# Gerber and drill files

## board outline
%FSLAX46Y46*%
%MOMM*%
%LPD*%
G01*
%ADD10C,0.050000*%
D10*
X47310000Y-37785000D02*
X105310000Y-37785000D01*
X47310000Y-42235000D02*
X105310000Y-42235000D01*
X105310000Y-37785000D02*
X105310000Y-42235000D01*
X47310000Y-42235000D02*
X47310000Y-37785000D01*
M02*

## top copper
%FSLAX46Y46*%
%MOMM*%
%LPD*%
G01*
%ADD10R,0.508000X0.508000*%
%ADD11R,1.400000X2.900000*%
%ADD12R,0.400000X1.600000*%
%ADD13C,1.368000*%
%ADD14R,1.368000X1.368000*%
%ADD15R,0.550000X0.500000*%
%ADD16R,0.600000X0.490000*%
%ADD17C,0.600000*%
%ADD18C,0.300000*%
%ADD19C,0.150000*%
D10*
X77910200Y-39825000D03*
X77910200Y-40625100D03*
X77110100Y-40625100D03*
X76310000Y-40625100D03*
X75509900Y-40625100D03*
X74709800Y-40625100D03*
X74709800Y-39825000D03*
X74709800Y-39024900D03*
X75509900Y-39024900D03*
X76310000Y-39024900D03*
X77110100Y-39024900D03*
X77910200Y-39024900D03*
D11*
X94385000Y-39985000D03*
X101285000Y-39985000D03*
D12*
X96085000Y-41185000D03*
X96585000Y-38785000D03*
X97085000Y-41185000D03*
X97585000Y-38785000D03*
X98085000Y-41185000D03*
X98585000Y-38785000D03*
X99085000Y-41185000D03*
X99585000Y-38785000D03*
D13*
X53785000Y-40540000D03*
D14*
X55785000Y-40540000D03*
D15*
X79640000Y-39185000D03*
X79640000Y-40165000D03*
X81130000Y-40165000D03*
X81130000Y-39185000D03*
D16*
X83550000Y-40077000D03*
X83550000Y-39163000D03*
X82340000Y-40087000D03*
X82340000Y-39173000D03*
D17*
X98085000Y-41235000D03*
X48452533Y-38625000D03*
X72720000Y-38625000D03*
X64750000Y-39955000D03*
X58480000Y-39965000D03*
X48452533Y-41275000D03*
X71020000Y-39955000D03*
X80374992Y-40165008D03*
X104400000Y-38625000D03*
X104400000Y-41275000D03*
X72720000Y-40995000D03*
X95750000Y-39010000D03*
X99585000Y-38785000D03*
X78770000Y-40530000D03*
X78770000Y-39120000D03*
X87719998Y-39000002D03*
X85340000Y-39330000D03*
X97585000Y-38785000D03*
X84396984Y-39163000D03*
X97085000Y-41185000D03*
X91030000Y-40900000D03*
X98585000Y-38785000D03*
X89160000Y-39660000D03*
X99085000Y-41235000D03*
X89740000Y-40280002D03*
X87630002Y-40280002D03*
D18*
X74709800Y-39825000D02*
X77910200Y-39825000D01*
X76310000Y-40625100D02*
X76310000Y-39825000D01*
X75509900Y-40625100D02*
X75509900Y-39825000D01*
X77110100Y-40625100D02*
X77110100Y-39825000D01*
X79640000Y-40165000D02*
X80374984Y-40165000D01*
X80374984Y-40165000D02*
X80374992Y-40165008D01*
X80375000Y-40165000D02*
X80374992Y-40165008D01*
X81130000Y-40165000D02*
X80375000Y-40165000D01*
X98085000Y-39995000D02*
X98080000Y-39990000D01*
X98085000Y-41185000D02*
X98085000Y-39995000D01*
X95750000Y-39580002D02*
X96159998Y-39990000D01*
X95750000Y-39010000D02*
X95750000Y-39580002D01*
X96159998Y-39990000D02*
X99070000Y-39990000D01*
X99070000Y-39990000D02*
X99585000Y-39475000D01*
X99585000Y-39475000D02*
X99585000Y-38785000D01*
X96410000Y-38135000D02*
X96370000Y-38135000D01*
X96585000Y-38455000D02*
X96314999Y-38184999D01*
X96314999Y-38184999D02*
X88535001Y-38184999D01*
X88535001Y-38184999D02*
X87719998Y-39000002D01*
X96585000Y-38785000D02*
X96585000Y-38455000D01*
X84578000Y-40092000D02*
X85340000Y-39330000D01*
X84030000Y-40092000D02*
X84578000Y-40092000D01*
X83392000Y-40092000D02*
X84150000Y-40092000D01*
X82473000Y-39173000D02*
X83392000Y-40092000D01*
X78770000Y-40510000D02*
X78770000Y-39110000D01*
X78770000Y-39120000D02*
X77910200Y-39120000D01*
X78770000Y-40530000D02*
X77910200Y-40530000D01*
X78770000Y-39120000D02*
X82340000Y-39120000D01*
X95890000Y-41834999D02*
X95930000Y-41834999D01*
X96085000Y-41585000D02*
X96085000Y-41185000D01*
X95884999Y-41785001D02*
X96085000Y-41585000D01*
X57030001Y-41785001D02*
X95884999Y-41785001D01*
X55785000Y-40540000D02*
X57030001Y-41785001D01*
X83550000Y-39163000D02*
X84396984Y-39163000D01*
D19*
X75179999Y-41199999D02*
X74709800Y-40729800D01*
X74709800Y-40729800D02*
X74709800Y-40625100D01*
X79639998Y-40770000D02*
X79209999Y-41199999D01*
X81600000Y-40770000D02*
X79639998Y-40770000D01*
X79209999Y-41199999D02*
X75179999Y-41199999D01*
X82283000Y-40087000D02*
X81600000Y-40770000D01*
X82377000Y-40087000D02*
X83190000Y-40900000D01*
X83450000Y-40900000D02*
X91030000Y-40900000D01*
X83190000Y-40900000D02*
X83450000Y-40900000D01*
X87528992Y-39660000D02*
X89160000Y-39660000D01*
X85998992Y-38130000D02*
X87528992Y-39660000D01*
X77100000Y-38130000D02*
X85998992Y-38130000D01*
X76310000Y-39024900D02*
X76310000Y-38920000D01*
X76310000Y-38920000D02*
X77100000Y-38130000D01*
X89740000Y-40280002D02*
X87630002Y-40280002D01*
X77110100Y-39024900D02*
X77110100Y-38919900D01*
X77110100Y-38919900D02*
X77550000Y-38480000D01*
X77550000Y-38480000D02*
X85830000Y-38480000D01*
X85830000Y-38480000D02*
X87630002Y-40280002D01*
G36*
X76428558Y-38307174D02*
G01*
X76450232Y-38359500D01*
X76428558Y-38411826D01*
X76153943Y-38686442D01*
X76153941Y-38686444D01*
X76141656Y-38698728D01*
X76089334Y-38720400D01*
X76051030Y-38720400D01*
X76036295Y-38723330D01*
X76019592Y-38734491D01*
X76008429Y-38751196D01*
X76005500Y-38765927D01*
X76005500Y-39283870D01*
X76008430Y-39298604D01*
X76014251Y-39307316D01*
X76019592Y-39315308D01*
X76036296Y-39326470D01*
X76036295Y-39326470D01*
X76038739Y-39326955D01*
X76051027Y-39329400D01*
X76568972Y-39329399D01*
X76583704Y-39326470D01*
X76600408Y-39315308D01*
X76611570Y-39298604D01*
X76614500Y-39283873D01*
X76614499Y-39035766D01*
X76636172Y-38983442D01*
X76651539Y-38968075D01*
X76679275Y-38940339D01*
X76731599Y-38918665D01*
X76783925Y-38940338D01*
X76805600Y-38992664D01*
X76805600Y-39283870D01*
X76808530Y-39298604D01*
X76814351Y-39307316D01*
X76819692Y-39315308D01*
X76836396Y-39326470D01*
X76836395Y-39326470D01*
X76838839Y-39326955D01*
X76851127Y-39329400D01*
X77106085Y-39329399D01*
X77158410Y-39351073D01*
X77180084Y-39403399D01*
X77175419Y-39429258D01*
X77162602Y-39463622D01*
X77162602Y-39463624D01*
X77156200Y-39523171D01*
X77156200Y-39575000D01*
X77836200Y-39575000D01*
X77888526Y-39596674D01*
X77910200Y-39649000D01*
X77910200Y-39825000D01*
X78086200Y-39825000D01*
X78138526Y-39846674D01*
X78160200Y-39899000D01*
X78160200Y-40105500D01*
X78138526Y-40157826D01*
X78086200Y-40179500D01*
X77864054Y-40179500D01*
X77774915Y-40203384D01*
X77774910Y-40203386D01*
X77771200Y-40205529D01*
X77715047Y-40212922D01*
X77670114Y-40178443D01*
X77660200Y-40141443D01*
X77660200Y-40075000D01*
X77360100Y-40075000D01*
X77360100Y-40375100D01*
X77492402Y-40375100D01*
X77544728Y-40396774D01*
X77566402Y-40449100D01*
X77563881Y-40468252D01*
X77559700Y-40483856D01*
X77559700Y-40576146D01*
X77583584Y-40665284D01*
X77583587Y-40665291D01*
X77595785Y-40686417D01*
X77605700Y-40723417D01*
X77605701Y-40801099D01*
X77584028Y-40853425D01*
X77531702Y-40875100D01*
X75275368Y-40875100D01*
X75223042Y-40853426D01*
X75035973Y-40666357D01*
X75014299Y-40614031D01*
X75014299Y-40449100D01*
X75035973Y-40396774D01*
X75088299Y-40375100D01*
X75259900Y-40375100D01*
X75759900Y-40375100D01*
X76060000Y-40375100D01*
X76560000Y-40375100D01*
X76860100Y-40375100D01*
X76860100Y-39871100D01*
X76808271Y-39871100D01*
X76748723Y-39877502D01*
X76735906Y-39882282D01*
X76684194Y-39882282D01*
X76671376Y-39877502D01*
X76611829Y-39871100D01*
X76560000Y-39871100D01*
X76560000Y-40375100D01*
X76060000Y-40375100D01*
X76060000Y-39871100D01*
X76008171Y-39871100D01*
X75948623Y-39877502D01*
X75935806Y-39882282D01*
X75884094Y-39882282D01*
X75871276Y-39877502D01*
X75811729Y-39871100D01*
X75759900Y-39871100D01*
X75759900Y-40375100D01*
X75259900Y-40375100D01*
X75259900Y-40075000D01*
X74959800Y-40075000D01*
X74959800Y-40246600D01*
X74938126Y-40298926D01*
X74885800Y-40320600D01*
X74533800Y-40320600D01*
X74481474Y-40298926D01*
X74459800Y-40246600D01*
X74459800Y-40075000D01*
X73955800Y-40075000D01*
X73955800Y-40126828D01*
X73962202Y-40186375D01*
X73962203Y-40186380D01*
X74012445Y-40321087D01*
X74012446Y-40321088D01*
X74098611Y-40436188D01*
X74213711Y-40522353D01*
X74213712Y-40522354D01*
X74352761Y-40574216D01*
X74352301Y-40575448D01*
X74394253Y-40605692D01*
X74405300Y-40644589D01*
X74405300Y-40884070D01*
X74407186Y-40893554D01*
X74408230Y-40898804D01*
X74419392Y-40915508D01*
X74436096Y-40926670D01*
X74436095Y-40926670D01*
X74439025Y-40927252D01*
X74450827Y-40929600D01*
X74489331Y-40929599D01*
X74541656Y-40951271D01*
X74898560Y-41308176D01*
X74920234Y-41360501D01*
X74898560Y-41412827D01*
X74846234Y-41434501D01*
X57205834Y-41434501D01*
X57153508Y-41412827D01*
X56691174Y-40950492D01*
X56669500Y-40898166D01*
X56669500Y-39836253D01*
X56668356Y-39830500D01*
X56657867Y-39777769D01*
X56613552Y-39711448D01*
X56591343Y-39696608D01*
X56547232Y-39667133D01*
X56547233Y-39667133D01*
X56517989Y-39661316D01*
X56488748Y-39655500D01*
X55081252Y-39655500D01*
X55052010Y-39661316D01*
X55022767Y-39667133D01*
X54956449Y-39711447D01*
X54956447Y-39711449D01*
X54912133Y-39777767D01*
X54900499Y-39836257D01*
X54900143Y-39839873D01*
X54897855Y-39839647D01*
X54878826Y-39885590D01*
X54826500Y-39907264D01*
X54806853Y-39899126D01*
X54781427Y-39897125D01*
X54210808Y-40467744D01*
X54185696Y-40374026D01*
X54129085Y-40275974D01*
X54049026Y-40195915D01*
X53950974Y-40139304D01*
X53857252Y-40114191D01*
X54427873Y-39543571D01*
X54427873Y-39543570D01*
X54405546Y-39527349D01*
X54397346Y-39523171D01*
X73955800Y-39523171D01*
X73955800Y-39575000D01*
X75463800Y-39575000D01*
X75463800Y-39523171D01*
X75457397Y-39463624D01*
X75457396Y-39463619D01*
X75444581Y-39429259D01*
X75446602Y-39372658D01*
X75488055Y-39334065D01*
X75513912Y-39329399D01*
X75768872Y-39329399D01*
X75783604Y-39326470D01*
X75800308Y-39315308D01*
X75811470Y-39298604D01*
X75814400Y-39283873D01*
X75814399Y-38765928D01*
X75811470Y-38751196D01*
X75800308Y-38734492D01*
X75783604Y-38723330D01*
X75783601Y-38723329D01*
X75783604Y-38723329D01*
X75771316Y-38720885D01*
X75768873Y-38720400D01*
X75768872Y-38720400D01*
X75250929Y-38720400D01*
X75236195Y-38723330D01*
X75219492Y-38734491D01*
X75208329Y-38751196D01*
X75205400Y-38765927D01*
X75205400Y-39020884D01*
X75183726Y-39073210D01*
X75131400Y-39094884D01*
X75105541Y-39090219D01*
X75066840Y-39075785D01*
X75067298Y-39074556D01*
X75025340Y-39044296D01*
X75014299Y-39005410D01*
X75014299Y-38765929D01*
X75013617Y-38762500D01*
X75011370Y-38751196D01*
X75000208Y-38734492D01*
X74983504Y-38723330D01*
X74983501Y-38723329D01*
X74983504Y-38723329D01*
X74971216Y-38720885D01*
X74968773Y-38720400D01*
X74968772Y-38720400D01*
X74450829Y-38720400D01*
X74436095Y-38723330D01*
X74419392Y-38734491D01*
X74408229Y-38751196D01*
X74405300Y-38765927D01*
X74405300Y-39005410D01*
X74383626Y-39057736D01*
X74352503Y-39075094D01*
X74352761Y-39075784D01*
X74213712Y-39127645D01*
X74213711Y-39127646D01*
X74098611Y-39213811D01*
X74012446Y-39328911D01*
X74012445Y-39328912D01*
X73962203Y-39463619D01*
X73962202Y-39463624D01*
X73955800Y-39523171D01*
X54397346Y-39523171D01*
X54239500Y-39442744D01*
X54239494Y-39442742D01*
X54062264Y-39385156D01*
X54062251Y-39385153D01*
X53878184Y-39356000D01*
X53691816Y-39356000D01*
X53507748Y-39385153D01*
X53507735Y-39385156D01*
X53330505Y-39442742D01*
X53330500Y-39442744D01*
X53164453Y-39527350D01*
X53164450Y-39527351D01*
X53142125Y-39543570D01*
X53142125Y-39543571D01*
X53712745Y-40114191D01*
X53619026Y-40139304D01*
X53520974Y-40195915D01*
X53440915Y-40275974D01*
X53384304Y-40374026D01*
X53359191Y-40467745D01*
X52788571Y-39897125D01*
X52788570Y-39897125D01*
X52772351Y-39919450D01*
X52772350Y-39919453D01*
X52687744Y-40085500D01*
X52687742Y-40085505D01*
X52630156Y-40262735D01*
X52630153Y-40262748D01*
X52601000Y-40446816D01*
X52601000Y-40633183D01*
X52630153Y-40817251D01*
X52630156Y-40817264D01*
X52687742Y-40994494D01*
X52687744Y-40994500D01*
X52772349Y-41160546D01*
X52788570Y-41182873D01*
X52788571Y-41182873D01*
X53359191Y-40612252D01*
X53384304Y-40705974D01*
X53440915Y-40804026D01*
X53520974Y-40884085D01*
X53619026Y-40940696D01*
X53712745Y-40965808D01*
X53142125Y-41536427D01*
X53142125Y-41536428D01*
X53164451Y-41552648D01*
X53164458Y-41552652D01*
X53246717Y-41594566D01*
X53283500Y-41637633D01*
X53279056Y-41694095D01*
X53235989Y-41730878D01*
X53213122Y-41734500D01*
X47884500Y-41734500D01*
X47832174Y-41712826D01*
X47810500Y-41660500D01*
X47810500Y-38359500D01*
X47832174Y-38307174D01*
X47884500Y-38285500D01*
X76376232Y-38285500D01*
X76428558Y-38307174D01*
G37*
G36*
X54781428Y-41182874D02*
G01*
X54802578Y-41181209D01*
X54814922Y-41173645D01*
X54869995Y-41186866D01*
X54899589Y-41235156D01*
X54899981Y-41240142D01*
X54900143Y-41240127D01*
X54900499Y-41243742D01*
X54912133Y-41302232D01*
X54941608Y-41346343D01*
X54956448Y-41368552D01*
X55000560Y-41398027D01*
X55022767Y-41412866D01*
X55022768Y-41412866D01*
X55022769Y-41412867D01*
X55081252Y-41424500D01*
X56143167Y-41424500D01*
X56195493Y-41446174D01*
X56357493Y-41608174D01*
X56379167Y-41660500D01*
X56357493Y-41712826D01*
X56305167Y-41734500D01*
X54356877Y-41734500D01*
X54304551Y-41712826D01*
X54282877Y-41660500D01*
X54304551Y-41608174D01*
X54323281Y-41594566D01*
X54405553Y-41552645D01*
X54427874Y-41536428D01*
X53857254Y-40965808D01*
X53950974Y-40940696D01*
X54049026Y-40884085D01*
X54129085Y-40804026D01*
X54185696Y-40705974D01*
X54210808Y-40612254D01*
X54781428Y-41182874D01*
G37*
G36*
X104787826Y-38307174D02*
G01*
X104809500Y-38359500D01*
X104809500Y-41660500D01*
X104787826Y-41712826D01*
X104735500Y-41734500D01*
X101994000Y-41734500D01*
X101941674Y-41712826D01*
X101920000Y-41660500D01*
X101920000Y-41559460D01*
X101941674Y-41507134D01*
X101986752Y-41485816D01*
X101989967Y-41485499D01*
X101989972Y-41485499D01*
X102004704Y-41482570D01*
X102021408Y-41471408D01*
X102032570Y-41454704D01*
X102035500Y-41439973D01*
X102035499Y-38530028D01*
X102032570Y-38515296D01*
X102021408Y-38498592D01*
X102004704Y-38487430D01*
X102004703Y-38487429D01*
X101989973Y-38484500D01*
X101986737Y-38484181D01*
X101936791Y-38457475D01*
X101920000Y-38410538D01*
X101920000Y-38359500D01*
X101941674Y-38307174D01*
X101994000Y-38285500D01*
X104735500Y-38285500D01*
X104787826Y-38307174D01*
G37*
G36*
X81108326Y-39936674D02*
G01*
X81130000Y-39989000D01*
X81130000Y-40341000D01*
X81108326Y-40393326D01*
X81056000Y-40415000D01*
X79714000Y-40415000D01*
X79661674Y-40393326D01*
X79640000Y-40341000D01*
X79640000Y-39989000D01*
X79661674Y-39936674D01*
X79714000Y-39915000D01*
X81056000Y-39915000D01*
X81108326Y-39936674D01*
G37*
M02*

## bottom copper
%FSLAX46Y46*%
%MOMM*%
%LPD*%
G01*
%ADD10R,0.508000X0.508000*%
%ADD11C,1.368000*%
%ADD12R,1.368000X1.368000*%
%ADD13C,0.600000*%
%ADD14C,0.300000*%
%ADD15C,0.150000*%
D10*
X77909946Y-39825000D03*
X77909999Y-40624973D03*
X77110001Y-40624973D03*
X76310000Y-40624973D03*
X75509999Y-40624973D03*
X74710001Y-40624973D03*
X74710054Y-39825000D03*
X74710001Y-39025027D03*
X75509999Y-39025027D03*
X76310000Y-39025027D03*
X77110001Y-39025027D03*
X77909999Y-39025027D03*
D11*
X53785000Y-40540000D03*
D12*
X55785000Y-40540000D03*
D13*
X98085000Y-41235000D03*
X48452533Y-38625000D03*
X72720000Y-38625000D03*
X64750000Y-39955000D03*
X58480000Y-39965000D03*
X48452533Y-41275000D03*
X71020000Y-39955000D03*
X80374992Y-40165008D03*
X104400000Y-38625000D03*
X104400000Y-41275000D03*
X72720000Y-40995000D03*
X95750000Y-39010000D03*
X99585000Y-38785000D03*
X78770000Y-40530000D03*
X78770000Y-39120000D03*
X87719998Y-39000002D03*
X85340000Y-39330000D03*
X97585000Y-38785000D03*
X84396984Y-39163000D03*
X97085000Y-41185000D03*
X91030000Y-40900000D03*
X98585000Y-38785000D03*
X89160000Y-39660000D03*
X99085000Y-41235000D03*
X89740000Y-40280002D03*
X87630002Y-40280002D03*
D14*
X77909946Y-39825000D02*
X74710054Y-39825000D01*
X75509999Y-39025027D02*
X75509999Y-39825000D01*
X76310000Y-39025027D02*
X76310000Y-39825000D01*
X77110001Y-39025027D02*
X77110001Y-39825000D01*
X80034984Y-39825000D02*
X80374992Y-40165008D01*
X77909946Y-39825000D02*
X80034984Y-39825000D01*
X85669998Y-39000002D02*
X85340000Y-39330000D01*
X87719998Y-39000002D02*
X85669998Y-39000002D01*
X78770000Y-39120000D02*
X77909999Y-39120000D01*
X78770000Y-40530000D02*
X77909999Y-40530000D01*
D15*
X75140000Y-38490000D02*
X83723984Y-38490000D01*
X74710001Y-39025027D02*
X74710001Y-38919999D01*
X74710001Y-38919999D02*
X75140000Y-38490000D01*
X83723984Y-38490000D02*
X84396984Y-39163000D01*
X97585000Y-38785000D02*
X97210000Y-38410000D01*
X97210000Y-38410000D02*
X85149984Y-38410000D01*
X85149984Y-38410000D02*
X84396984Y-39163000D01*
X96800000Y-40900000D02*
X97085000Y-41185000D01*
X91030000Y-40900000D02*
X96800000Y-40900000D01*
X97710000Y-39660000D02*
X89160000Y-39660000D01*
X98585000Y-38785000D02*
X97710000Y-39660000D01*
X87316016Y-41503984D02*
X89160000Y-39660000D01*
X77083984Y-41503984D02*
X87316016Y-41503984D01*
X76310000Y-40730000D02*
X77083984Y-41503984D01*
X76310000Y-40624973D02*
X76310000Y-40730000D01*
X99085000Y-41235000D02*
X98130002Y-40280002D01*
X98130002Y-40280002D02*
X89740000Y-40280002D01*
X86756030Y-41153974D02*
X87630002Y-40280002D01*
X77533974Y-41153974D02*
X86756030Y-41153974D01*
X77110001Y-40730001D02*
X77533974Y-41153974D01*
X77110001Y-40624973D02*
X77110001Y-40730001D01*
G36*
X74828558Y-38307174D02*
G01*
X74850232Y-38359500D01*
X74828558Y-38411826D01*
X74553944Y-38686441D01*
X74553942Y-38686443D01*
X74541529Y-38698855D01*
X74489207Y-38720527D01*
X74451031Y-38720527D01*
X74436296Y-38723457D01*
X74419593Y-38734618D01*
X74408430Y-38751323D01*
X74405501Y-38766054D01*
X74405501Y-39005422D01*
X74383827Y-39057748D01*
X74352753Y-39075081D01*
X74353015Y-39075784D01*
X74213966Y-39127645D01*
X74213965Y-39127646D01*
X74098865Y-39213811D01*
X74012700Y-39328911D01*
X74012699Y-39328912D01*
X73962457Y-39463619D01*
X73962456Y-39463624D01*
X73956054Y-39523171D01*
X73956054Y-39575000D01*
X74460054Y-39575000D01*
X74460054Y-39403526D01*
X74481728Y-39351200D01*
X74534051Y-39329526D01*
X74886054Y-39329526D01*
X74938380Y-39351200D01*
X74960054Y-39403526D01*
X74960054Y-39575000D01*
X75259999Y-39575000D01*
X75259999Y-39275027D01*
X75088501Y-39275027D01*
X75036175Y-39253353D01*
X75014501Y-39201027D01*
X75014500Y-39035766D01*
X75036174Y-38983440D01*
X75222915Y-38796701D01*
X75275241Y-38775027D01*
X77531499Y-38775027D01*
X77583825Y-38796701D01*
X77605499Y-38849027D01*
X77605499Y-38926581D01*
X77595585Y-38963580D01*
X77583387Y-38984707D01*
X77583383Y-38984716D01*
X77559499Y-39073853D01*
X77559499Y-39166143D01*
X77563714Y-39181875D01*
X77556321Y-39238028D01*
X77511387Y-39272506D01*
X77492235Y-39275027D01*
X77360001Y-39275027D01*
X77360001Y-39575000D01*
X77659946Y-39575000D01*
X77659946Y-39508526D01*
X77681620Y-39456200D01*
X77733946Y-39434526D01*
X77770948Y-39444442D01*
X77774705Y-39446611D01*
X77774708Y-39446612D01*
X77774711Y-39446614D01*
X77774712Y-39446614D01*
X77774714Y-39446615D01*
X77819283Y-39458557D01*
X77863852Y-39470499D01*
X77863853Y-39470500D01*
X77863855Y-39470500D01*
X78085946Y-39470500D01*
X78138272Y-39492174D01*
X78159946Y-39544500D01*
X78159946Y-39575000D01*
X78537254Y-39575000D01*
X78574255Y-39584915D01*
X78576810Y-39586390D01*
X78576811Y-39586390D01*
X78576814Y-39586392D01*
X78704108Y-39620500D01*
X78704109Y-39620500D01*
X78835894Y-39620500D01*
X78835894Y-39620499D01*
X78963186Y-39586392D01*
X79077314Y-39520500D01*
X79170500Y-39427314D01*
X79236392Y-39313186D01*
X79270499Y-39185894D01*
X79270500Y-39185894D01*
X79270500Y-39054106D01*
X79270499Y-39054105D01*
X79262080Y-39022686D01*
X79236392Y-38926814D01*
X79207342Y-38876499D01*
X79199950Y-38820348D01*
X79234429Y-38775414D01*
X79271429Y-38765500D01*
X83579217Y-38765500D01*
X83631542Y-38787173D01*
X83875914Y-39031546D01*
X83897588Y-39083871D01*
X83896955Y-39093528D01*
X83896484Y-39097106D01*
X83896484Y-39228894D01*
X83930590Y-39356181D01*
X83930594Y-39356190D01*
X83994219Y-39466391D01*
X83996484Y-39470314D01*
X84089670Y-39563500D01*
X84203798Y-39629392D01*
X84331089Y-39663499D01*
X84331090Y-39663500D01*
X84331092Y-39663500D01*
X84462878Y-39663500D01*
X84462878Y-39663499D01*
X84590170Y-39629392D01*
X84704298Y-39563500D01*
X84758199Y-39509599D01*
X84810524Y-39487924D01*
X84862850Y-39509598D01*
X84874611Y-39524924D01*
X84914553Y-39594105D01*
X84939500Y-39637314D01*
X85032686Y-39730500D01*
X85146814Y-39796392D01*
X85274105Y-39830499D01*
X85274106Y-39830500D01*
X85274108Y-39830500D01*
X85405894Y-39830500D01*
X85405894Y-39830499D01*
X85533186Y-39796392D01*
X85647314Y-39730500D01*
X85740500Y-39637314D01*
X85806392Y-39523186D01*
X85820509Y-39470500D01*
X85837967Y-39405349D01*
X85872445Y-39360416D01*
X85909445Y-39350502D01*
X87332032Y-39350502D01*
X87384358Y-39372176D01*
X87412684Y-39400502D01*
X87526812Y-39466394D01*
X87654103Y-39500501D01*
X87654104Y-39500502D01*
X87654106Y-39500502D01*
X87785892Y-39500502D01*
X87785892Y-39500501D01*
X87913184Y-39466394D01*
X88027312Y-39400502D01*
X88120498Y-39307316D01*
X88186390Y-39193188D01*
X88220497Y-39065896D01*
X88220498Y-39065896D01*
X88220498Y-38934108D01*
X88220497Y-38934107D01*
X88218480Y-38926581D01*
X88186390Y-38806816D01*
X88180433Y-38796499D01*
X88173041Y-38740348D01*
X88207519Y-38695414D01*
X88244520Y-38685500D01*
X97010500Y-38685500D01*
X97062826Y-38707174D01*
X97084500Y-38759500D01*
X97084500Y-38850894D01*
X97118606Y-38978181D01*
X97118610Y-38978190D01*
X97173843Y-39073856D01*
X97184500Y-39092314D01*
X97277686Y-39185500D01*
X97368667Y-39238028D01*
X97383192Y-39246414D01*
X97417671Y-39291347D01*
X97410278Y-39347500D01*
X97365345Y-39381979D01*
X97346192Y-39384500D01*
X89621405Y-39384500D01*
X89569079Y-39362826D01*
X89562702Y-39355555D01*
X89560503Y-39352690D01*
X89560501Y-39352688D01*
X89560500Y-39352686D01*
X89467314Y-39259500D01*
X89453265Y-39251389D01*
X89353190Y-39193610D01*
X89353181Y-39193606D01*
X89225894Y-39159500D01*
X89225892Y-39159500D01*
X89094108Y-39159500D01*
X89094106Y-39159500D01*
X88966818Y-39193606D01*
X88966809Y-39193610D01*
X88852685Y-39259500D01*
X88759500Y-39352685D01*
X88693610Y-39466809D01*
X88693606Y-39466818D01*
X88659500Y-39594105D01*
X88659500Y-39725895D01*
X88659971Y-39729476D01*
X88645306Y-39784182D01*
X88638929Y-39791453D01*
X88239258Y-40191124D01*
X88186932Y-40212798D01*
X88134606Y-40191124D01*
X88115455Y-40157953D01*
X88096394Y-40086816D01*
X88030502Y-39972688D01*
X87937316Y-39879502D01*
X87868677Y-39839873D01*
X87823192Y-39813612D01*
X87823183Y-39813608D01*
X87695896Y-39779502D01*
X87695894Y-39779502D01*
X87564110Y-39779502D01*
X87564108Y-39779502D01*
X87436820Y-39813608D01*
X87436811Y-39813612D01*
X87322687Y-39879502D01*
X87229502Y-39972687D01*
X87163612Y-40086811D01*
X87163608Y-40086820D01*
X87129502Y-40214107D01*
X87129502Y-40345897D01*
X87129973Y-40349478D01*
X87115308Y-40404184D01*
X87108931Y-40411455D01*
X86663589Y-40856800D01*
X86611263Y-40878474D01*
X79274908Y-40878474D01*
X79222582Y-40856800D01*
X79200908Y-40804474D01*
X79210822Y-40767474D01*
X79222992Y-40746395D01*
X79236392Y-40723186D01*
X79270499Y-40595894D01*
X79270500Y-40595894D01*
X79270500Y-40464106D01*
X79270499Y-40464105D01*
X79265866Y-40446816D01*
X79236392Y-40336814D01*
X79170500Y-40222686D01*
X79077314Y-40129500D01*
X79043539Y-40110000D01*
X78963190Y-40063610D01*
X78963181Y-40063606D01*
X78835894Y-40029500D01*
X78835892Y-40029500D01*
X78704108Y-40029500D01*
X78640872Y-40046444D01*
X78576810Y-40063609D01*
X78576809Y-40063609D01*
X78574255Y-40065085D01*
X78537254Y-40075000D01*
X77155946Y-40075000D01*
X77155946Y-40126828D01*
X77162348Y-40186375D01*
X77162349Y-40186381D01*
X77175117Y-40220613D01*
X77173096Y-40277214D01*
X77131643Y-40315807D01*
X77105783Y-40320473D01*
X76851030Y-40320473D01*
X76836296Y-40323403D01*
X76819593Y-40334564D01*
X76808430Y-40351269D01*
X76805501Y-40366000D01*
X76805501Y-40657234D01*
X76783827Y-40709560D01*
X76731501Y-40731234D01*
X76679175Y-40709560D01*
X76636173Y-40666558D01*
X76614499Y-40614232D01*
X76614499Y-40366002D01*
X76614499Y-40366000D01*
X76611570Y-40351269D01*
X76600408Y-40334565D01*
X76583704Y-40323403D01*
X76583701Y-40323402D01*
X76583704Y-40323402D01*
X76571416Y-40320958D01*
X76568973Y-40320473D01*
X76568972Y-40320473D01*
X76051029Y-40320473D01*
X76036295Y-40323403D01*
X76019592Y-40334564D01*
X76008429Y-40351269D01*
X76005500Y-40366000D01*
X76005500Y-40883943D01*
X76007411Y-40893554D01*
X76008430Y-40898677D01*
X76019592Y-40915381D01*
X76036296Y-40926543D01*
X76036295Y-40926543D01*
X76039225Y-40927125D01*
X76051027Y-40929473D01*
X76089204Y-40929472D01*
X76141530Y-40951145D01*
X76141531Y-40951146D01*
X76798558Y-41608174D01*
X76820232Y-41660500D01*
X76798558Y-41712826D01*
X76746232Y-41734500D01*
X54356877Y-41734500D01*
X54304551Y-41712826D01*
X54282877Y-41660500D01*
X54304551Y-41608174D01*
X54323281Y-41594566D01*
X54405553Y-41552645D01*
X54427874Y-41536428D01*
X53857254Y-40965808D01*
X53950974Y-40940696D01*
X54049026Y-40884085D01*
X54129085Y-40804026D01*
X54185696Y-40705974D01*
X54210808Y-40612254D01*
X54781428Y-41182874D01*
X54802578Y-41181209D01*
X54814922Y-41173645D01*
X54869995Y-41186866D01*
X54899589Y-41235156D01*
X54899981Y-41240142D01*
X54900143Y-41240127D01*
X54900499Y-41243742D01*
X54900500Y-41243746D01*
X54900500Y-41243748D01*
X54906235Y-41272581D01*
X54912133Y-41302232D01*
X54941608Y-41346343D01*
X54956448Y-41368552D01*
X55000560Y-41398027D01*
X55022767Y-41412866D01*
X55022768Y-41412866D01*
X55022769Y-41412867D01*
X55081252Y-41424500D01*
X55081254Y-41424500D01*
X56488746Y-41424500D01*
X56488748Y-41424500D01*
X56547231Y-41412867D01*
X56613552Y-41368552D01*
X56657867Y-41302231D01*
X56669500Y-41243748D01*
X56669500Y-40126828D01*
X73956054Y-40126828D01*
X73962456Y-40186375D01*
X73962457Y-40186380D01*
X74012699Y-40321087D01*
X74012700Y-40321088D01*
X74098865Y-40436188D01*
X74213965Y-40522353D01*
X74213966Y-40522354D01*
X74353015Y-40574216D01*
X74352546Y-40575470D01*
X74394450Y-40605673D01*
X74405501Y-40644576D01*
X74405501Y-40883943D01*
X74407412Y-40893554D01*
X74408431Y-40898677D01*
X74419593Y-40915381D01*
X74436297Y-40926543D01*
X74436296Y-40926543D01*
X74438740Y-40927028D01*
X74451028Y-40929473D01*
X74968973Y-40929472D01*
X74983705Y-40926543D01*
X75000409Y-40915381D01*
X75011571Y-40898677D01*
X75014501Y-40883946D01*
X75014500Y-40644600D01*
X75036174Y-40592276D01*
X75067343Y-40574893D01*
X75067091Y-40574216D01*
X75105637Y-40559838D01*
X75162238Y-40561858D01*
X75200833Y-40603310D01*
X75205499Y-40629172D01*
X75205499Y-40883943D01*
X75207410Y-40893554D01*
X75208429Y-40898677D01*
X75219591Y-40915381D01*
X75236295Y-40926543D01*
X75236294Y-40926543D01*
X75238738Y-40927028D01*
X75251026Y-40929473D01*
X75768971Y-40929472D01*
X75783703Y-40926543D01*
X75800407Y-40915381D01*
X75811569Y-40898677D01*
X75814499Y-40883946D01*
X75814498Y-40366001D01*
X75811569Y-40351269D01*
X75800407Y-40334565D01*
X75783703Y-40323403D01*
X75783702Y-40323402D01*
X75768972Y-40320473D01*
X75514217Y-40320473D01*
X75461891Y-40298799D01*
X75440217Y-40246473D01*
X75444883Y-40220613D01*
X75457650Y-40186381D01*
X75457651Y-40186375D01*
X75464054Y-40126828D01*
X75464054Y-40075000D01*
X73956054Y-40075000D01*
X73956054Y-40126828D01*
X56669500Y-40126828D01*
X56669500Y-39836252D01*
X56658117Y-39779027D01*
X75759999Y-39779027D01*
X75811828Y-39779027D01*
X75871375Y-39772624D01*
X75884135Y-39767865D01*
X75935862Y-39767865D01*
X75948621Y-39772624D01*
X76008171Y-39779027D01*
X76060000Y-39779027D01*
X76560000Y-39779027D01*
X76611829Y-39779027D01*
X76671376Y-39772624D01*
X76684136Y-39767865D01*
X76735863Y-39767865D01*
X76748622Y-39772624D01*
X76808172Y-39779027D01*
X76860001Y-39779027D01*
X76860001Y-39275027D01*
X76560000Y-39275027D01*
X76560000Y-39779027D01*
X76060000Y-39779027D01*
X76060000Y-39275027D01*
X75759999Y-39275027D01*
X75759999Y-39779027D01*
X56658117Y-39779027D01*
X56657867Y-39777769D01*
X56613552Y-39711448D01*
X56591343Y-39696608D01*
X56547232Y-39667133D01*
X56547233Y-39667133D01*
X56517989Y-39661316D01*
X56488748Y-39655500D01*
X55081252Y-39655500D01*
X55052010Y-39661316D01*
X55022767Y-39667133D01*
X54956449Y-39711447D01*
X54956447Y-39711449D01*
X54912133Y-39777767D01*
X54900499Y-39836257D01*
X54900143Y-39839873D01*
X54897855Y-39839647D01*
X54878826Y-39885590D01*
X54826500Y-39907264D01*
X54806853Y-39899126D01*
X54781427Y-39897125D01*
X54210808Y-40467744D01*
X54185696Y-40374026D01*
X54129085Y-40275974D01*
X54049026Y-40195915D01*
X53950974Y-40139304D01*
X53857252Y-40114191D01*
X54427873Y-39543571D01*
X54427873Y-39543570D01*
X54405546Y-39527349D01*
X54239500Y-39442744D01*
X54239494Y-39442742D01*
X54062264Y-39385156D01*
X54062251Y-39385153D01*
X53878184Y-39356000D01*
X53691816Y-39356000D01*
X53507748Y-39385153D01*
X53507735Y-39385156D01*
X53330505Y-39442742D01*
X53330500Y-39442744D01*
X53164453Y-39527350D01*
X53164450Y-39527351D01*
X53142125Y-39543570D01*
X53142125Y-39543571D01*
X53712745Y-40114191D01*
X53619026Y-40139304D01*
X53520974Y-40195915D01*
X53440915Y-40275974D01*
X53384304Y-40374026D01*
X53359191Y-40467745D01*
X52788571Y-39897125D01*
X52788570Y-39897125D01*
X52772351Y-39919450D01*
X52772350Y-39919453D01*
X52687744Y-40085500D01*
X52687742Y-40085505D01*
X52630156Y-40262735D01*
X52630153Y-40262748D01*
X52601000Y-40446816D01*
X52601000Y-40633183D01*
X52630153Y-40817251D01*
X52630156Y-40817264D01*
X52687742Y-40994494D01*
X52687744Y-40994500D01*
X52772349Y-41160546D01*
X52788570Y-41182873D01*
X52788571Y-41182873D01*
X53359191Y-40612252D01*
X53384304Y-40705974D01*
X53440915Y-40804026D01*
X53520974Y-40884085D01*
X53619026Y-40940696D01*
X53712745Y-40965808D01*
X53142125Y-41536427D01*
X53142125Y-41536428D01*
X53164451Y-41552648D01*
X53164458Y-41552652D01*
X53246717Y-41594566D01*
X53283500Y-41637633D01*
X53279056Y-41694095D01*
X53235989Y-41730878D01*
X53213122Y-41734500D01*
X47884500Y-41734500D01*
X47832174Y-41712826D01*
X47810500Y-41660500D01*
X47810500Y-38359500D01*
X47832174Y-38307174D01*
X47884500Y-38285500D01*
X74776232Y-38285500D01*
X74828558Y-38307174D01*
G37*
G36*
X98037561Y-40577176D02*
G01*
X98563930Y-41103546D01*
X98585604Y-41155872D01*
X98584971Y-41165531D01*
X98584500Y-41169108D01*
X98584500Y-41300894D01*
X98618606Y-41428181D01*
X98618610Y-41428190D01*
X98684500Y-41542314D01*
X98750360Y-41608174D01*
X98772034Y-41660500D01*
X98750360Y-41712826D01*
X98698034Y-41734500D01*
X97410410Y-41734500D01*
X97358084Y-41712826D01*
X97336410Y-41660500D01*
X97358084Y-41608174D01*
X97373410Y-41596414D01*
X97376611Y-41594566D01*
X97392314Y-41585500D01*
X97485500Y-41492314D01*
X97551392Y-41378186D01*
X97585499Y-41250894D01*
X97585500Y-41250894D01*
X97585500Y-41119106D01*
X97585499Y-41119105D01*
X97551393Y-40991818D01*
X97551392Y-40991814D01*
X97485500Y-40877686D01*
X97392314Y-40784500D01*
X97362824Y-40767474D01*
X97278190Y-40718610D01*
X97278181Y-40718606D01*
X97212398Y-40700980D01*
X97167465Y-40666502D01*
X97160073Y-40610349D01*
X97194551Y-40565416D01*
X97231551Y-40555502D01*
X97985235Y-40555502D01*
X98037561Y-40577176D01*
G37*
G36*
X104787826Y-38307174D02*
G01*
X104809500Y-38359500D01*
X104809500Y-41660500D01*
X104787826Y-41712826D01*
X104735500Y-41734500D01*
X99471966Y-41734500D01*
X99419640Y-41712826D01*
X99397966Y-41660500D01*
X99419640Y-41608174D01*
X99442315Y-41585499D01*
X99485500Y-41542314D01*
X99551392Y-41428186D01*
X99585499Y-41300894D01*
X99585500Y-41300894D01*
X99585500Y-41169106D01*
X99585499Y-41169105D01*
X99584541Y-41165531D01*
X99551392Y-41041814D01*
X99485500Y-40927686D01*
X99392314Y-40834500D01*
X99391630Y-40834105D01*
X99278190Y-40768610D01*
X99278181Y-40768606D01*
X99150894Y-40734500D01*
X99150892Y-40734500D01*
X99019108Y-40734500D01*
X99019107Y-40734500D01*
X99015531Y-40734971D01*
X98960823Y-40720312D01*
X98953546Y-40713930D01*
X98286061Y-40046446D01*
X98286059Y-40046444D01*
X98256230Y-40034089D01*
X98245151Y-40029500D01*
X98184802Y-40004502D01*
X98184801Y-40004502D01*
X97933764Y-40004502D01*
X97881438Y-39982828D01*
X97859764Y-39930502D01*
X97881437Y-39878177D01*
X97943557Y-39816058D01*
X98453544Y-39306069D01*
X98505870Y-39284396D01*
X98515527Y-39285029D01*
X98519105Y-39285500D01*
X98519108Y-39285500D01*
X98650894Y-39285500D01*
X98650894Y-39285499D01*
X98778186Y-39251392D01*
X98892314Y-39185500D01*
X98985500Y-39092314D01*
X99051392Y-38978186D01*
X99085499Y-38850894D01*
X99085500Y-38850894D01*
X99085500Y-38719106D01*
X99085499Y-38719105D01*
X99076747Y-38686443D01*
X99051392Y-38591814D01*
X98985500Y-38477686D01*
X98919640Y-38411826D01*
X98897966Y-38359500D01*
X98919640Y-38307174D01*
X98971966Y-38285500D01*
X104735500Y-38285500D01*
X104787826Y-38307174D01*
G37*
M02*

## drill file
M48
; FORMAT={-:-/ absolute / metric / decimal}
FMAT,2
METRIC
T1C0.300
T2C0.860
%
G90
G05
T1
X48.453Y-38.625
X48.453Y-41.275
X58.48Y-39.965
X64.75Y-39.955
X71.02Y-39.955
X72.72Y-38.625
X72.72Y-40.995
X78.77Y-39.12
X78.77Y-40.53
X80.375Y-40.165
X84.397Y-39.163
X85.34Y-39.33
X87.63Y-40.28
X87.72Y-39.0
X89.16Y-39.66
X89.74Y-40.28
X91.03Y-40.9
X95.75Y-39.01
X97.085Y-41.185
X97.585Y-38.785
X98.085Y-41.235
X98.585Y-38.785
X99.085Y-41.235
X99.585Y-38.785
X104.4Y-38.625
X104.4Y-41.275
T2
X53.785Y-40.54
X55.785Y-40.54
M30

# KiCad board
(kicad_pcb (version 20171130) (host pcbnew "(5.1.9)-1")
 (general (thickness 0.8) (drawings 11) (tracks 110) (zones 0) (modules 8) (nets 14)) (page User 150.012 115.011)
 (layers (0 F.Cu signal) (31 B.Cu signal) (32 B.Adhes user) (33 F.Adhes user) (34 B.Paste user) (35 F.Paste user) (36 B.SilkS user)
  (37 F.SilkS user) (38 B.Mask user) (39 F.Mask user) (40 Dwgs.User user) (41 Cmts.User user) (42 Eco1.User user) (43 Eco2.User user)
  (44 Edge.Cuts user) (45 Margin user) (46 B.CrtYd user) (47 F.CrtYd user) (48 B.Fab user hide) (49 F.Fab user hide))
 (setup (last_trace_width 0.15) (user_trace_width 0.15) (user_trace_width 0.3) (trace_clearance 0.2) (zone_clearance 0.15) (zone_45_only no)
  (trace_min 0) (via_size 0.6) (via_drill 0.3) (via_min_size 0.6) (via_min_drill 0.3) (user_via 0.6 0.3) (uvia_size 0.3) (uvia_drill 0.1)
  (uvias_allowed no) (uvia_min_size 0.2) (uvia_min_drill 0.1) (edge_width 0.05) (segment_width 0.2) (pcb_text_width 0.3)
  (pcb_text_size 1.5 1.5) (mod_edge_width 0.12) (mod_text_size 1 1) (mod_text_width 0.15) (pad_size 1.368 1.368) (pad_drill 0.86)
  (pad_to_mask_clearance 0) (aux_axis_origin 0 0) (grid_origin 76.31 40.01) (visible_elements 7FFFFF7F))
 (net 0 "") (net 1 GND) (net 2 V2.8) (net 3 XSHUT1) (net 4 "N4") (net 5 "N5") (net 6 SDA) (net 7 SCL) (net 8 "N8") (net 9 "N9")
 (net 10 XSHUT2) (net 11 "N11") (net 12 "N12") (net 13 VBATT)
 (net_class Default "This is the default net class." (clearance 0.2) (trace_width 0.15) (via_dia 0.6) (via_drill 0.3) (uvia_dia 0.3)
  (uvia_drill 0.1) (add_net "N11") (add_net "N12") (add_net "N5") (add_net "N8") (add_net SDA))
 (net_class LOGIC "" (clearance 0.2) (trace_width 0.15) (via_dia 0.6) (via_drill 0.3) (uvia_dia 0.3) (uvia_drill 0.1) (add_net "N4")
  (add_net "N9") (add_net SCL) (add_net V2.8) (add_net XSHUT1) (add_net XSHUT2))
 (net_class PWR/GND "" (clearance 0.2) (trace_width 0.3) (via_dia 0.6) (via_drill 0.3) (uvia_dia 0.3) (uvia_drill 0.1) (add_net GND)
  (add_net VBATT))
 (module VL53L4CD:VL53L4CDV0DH (layer F.Cu) (at 76.31 39.825 270) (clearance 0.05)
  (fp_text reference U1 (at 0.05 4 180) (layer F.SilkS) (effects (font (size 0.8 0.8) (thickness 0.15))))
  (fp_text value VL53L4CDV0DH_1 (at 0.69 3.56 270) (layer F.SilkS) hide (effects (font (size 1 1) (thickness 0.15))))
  (pad 12 smd rect (at 0 -1.6002 270) (size 0.508 0.508) (layers F.Cu F.Mask) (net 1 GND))
  (pad 1 smd rect (at 0.8001 -1.6002) (size 0.508 0.508) (layers F.Cu F.Mask) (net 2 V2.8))
  (pad 2 smd rect (at 0.8001 -0.8001) (size 0.508 0.508) (layers F.Cu F.Mask) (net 1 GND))
  (pad 3 smd rect (at 0.8001 0) (size 0.508 0.508) (layers F.Cu F.Mask) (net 1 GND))
  (pad 4 smd rect (at 0.8001 0.8001) (size 0.508 0.508) (layers F.Cu F.Mask) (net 1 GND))
  (pad 5 smd rect (at 0.8001 1.6002) (size 0.508 0.508) (layers F.Cu F.Mask) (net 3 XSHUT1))
  (pad 6 smd rect (at 0 1.6002 270) (size 0.508 0.508) (layers F.Cu F.Mask) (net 1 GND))
  (pad 7 smd rect (at -0.8001 1.6002) (size 0.508 0.508) (layers F.Cu F.Mask) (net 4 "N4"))
  (pad 8 smd rect (at -0.8001 0.8001) (size 0.508 0.508) (layers F.Cu F.Mask) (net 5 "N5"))
  (pad 9 smd rect (at -0.8001 0) (size 0.508 0.508) (layers F.Cu F.Mask) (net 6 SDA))
  (pad 10 smd rect (at -0.8001 -0.8001) (size 0.508 0.508) (layers F.Cu F.Mask) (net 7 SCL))
  (pad 11 smd rect (at -0.8001 -1.6002) (size 0.508 0.508) (layers F.Cu F.Mask) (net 2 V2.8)))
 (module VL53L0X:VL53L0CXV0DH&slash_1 (layer B.Cu) (at 76.31 39.825 90) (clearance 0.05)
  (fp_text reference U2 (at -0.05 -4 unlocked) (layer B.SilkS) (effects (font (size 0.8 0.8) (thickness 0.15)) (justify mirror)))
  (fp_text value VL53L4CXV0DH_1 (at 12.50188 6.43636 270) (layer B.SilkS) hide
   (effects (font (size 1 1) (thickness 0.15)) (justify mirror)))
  (pad 12 smd rect (at 0 1.599946 90) (size 0.508 0.508) (layers B.Cu B.Paste B.Mask) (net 1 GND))
  (pad 11 smd rect (at -0.799973 1.599999) (size 0.508 0.508) (layers B.Cu B.Paste B.Mask) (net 2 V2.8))
  (pad 10 smd rect (at -0.799973 0.800001) (size 0.508 0.508) (layers B.Cu B.Paste B.Mask) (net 7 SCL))
  (pad 9 smd rect (at -0.799973 0) (size 0.508 0.508) (layers B.Cu B.Paste B.Mask) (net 6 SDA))
  (pad 8 smd rect (at -0.799973 -0.800001) (size 0.508 0.508) (layers B.Cu B.Paste B.Mask) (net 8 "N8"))
  (pad 7 smd rect (at -0.799973 -1.599999) (size 0.508 0.508) (layers B.Cu B.Paste B.Mask) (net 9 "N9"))
  (pad 6 smd rect (at 0 -1.599946 90) (size 0.508 0.508) (layers B.Cu B.Paste B.Mask) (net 1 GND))
  (pad 5 smd rect (at 0.799973 -1.599999) (size 0.508 0.508) (layers B.Cu B.Paste B.Mask) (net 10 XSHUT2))
  (pad 4 smd rect (at 0.799973 -0.800001) (size 0.508 0.508) (layers B.Cu B.Paste B.Mask) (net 1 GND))
  (pad 3 smd rect (at 0.799973 0) (size 0.508 0.508) (layers B.Cu B.Paste B.Mask) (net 1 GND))
  (pad 2 smd rect (at 0.799973 0.800001) (size 0.508 0.508) (layers B.Cu B.Paste B.Mask) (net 1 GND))
  (pad 1 smd rect (at 0.799973 1.599999) (size 0.508 0.508) (layers B.Cu B.Paste B.Mask) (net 2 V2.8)))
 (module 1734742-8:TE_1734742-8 (layer F.Cu) (at 97.835 39.985) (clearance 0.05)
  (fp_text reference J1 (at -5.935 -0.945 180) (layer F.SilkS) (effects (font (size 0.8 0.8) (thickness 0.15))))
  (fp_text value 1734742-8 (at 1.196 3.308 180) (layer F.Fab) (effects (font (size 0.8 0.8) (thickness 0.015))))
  (pad S1 smd rect (at -3.45 0) (size 1.4 2.9) (layers F.Cu F.Paste F.Mask) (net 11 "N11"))
  (pad S2 smd rect (at 3.45 0) (size 1.4 2.9) (layers F.Cu F.Paste F.Mask) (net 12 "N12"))
  (pad 1 smd rect (at -1.75 1.2) (size 0.4 1.6) (layers F.Cu F.Paste F.Mask) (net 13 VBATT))
  (pad 2 smd rect (at -1.25 -1.2) (size 0.4 1.6) (layers F.Cu F.Paste F.Mask) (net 2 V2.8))
  (pad 3 smd rect (at -0.75 1.2) (size 0.4 1.6) (layers F.Cu F.Paste F.Mask) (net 3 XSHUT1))
  (pad 4 smd rect (at -0.25 -1.2) (size 0.4 1.6) (layers F.Cu F.Paste F.Mask) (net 10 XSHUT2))
  (pad 5 smd rect (at 0.25 1.2) (size 0.4 1.6) (layers F.Cu F.Paste F.Mask) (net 1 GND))
  (pad 6 smd rect (at 0.75 -1.2) (size 0.4 1.6) (layers F.Cu F.Paste F.Mask) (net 6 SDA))
  (pad 7 smd rect (at 1.25 1.2) (size 0.4 1.6) (layers F.Cu F.Paste F.Mask) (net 7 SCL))
  (pad 8 smd rect (at 1.75 -1.2) (size 0.4 1.6) (layers F.Cu F.Paste F.Mask) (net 1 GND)))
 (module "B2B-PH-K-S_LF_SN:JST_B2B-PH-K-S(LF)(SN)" (layer F.Cu) (at 54.785 39.99) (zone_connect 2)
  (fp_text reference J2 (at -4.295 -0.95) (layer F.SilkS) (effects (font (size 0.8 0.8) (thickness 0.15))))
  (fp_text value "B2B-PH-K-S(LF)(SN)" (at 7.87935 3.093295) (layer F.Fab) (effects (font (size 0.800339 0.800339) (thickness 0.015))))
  (pad 2 thru_hole circle (at -1 0.55) (size 1.368 1.368) (drill 0.86) (layers *.Cu *.Mask) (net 1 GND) (zone_connect 1))
  (pad 1 thru_hole rect (at 1 0.55) (size 1.368 1.368) (drill 0.86) (layers *.Cu *.Mask) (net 13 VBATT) (zone_connect 2)))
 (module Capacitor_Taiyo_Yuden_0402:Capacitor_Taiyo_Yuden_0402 (layer F.Cu) (at 79.64 39.675 270) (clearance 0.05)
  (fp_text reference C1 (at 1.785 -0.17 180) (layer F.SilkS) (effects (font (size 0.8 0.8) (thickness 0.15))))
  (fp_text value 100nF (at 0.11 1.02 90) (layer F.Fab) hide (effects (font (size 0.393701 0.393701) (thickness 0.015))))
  (pad 1 smd rect (at -0.49 0 270) (size 0.5 0.55) (layers F.Cu F.Paste F.Mask) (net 2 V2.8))
  (pad 2 smd rect (at 0.49 0 270) (size 0.5 0.55) (layers F.Cu F.Paste F.Mask) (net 1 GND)))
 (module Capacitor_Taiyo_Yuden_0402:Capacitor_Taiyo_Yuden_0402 (layer F.Cu) (at 81.13 39.675 270) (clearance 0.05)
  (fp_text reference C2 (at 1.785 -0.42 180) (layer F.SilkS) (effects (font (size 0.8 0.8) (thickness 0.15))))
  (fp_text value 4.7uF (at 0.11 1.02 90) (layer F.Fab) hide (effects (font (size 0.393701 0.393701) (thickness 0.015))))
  (pad 2 smd rect (at 0.49 0 270) (size 0.5 0.55) (layers F.Cu F.Paste F.Mask) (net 1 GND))
  (pad 1 smd rect (at -0.49 0 270) (size 0.5 0.55) (layers F.Cu F.Paste F.Mask) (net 2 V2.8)))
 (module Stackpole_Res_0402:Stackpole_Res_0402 (layer F.Cu) (at 83.55 39.62 270) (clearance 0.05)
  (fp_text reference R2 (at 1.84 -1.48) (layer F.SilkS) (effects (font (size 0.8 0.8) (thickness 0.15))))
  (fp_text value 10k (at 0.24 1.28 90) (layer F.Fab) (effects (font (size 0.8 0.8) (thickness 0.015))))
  (pad 2 smd rect (at 0.457 0 270) (size 0.49 0.6) (layers F.Cu F.Paste F.Mask) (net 2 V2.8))
  (pad 1 smd rect (at -0.457 0 270) (size 0.49 0.6) (layers F.Cu F.Paste F.Mask) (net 10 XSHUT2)))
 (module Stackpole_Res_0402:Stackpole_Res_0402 (layer F.Cu) (at 82.34 39.63 90) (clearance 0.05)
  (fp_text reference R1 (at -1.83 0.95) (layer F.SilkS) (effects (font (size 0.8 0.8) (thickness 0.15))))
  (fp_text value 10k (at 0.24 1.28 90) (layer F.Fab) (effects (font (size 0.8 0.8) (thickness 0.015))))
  (pad 1 smd rect (at -0.457 0 90) (size 0.49 0.6) (layers F.Cu F.Paste F.Mask) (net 3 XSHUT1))
  (pad 2 smd rect (at 0.457 0 90) (size 0.49 0.6) (layers F.Cu F.Paste F.Mask) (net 2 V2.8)))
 (gr_line (start 47.31 37.785) (end 105.31 37.785) (layer Edge.Cuts) (width 0.05))
 (gr_line (start 47.31 42.235) (end 105.31 42.235) (layer Edge.Cuts) (width 0.05))
 (gr_line (start 105.31 37.785) (end 105.31 42.235) (layer Edge.Cuts) (width 0.05))
 (gr_line (start 47.31 42.235) (end 47.31 37.785) (layer Edge.Cuts) (width 0.05))
 (via (at 98.085 41.235) (size 0.6) (drill 0.3) (layers F.Cu B.Cu) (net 1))
 (via (at 48.452533 38.625) (size 0.6) (drill 0.3) (layers F.Cu B.Cu) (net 1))
 (via (at 72.72 38.625) (size 0.6) (drill 0.3) (layers F.Cu B.Cu) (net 1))
 (via (at 64.75 39.955) (size 0.6) (drill 0.3) (layers F.Cu B.Cu) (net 1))
 (via (at 58.48 39.965) (size 0.6) (drill 0.3) (layers F.Cu B.Cu) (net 1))
 (via (at 48.452533 41.275) (size 0.6) (drill 0.3) (layers F.Cu B.Cu) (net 1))
 (via (at 71.02 39.955) (size 0.6) (drill 0.3) (layers F.Cu B.Cu) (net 1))
 (segment (start 74.7098 39.825) (end 77.9102 39.825) (width 0.3) (layer F.Cu) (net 1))
 (segment (start 77.909946 39.825) (end 74.710054 39.825) (width 0.3) (layer B.Cu) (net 1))
 (segment (start 75.509999 39.025027) (end 75.509999 39.825) (width 0.3) (layer B.Cu) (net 1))
 (segment (start 76.31 39.025027) (end 76.31 39.825) (width 0.3) (layer B.Cu) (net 1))
 (segment (start 77.110001 39.025027) (end 77.110001 39.825) (width 0.3) (layer B.Cu) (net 1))
 (segment (start 76.31 40.6251) (end 76.31 39.825) (width 0.3) (layer F.Cu) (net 1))
 (segment (start 75.5099 40.6251) (end 75.5099 39.825) (width 0.3) (layer F.Cu) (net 1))
 (segment (start 77.1101 40.6251) (end 77.1101 39.825) (width 0.3) (layer F.Cu) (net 1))
 (via (at 80.374992 40.165008) (size 0.6) (drill 0.3) (layers F.Cu B.Cu) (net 1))
 (segment (start 80.034984 39.825) (end 80.374992 40.165008) (width 0.3) (layer B.Cu) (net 1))
 (segment (start 77.909946 39.825) (end 80.034984 39.825) (width 0.3) (layer B.Cu) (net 1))
 (segment (start 79.64 40.165) (end 80.374984 40.165) (width 0.3) (layer F.Cu) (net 1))
 (segment (start 80.374984 40.165) (end 80.374992 40.165008) (width 0.3) (layer F.Cu) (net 1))
 (segment (start 80.375 40.165) (end 80.374992 40.165008) (width 0.3) (layer F.Cu) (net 1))
 (segment (start 81.13 40.165) (end 80.375 40.165) (width 0.3) (layer F.Cu) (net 1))
 (via (at 104.4 38.625) (size 0.6) (drill 0.3) (layers F.Cu B.Cu) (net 1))
 (via (at 104.4 41.275) (size 0.6) (drill 0.3) (layers F.Cu B.Cu) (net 1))
 (via (at 72.72 40.995) (size 0.6) (drill 0.3) (layers F.Cu B.Cu) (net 1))
 (via (at 95.75 39.01) (size 0.6) (drill 0.3) (layers F.Cu B.Cu) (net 1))
 (segment (start 98.085 39.995) (end 98.08 39.99) (width 0.3) (layer F.Cu) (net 1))
 (segment (start 98.085 41.185) (end 98.085 39.995) (width 0.3) (layer F.Cu) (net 1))
 (via (at 99.585 38.785) (size 0.6) (drill 0.3) (layers F.Cu B.Cu) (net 1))
 (segment (start 95.75 39.580002) (end 96.159998 39.99) (width 0.3) (layer F.Cu) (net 1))
 (segment (start 95.75 39.01) (end 95.75 39.580002) (width 0.3) (layer F.Cu) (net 1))
 (segment (start 96.159998 39.99) (end 99.07 39.99) (width 0.3) (layer F.Cu) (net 1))
 (segment (start 99.07 39.99) (end 99.585 39.475) (width 0.3) (layer F.Cu) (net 1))
 (segment (start 99.585 39.475) (end 99.585 38.785) (width 0.3) (layer F.Cu) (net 1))
 (segment (start 96.41 38.135) (end 96.37 38.135) (width 0.3) (layer F.Cu) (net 2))
 (via (at 78.77 40.53) (size 0.6) (drill 0.3) (layers F.Cu B.Cu) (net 2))
 (via (at 78.77 39.12) (size 0.6) (drill 0.3) (layers F.Cu B.Cu) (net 2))
 (segment (start 96.585 38.455) (end 96.314999 38.184999) (width 0.3) (layer F.Cu) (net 2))
 (segment (start 96.314999 38.184999) (end 88.535001 38.184999) (width 0.3) (layer F.Cu) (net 2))
 (segment (start 88.535001 38.184999) (end 87.719998 39.000002) (width 0.3) (layer F.Cu) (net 2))
 (segment (start 96.585 38.785) (end 96.585 38.455) (width 0.3) (layer F.Cu) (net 2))
 (via (at 87.719998 39.000002) (size 0.6) (drill 0.3) (layers F.Cu B.Cu) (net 2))
 (via (at 85.34 39.33) (size 0.6) (drill 0.3) (layers F.Cu B.Cu) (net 2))
 (segment (start 85.669998 39.000002) (end 85.34 39.33) (width 0.3) (layer B.Cu) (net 2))
 (segment (start 87.719998 39.000002) (end 85.669998 39.000002) (width 0.3) (layer B.Cu) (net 2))
 (segment (start 84.578 40.092) (end 85.34 39.33) (width 0.3) (layer F.Cu) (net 2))
 (segment (start 84.03 40.092) (end 84.578 40.092) (width 0.3) (layer F.Cu) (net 2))
 (segment (start 83.392 40.092) (end 84.15 40.092) (width 0.3) (layer F.Cu) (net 2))
 (segment (start 82.473 39.173) (end 83.392 40.092) (width 0.3) (layer F.Cu) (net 2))
 (segment (start 78.77 40.51) (end 78.77 39.11) (width 0.3) (layer F.Cu) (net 2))
 (segment (start 78.77 39.12) (end 77.909999 39.12) (width 0.3) (layer B.Cu) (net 2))
 (segment (start 78.77 40.53) (end 77.909999 40.53) (width 0.3) (layer B.Cu) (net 2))
 (segment (start 78.77 39.12) (end 77.9102 39.12) (width 0.3) (layer F.Cu) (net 2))
 (segment (start 78.77 40.53) (end 77.9102 40.53) (width 0.3) (layer F.Cu) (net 2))
 (segment (start 78.77 39.12) (end 82.34 39.12) (width 0.3) (layer F.Cu) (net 2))
 (segment (start 95.89 41.834999) (end 95.93 41.834999) (width 0.3) (layer F.Cu) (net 13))
 (segment (start 96.085 41.585) (end 96.085 41.185) (width 0.3) (layer F.Cu) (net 13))
 (segment (start 95.884999 41.785001) (end 96.085 41.585) (width 0.3) (layer F.Cu) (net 13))
 (segment (start 57.030001 41.785001) (end 95.884999 41.785001) (width 0.3) (layer F.Cu) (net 13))
 (segment (start 55.785 40.54) (end 57.030001 41.785001) (width 0.3) (layer F.Cu) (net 13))
 (via (at 97.585 38.785) (size 0.6) (drill 0.3) (layers F.Cu B.Cu) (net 10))
 (via (at 84.396984 39.163) (size 0.6) (drill 0.3) (layers F.Cu B.Cu) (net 10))
 (segment (start 75.14 38.49) (end 83.723984 38.49) (width 0.15) (layer B.Cu) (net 10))
 (segment (start 74.710001 39.025027) (end 74.710001 38.919999) (width 0.15) (layer B.Cu) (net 10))
 (segment (start 74.710001 38.919999) (end 75.14 38.49) (width 0.15) (layer B.Cu) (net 10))
 (segment (start 83.723984 38.49) (end 84.396984 39.163) (width 0.15) (layer B.Cu) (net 10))
 (segment (start 97.585 38.785) (end 97.21 38.41) (width 0.15) (layer B.Cu) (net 10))
 (segment (start 97.21 38.41) (end 85.149984 38.41) (width 0.15) (layer B.Cu) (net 10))
 (segment (start 85.149984 38.41) (end 84.396984 39.163) (width 0.15) (layer B.Cu) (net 10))
 (segment (start 83.55 39.163) (end 84.396984 39.163) (width 0.3) (layer F.Cu) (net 10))
 (via (at 97.085 41.185) (size 0.6) (drill 0.3) (layers F.Cu B.Cu) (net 3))
 (via (at 91.03 40.9) (size 0.6) (drill 0.3) (layers F.Cu B.Cu) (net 3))
 (segment (start 96.8 40.9) (end 97.085 41.185) (width 0.15) (layer B.Cu) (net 3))
 (segment (start 91.03 40.9) (end 96.8 40.9) (width 0.15) (layer B.Cu) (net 3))
 (segment (start 75.179999 41.199999) (end 74.7098 40.7298) (width 0.15) (layer F.Cu) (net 3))
 (segment (start 74.7098 40.7298) (end 74.7098 40.6251) (width 0.15) (layer F.Cu) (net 3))
 (segment (start 79.639998 40.77) (end 79.209999 41.199999) (width 0.15) (layer F.Cu) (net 3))
 (segment (start 81.6 40.77) (end 79.639998 40.77) (width 0.15) (layer F.Cu) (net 3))
 (segment (start 79.209999 41.199999) (end 75.179999 41.199999) (width 0.15) (layer F.Cu) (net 3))
 (segment (start 82.283 40.087) (end 81.6 40.77) (width 0.15) (layer F.Cu) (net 3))
 (segment (start 82.377 40.087) (end 83.19 40.9) (width 0.15) (layer F.Cu) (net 3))
 (segment (start 83.45 40.9) (end 91.03 40.9) (width 0.15) (layer F.Cu) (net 3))
 (segment (start 83.19 40.9) (end 83.45 40.9) (width 0.15) (layer F.Cu) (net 3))
 (via (at 98.585 38.785) (size 0.6) (drill 0.3) (layers F.Cu B.Cu) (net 6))
 (via (at 89.16 39.66) (size 0.6) (drill 0.3) (layers F.Cu B.Cu) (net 6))
 (segment (start 97.71 39.66) (end 89.16 39.66) (width 0.15) (layer B.Cu) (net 6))
 (segment (start 98.585 38.785) (end 97.71 39.66) (width 0.15) (layer B.Cu) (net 6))
 (segment (start 87.316016 41.503984) (end 89.16 39.66) (width 0.15) (layer B.Cu) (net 6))
 (segment (start 77.083984 41.503984) (end 87.316016 41.503984) (width 0.15) (layer B.Cu) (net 6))
 (segment (start 76.31 40.73) (end 77.083984 41.503984) (width 0.15) (layer B.Cu) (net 6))
 (segment (start 76.31 40.624973) (end 76.31 40.73) (width 0.15) (layer B.Cu) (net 6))
 (segment (start 87.528992 39.66) (end 89.16 39.66) (width 0.15) (layer F.Cu) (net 6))
 (segment (start 85.998992 38.13) (end 87.528992 39.66) (width 0.15) (layer F.Cu) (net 6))
 (segment (start 77.1 38.13) (end 85.998992 38.13) (width 0.15) (layer F.Cu) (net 6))
 (segment (start 76.31 39.0249) (end 76.31 38.92) (width 0.15) (layer F.Cu) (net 6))
 (segment (start 76.31 38.92) (end 77.1 38.13) (width 0.15) (layer F.Cu) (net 6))
 (via (at 99.085 41.235) (size 0.6) (drill 0.3) (layers F.Cu B.Cu) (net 7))
 (via (at 89.74 40.280002) (size 0.6) (drill 0.3) (layers F.Cu B.Cu) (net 7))
 (segment (start 99.085 41.235) (end 98.130002 40.280002) (width 0.15) (layer B.Cu) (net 7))
 (segment (start 98.130002 40.280002) (end 89.74 40.280002) (width 0.15) (layer B.Cu) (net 7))
 (via (at 87.630002 40.280002) (size 0.6) (drill 0.3) (layers F.Cu B.Cu) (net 7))
 (segment (start 89.74 40.280002) (end 87.630002 40.280002) (width 0.15) (layer F.Cu) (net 7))
 (segment (start 86.75603 41.153974) (end 87.630002 40.280002) (width 0.15) (layer B.Cu) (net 7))
 (segment (start 77.533974 41.153974) (end 86.75603 41.153974) (width 0.15) (layer B.Cu) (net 7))
 (segment (start 77.110001 40.730001) (end 77.533974 41.153974) (width 0.15) (layer B.Cu) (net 7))
 (segment (start 77.110001 40.624973) (end 77.110001 40.730001) (width 0.15) (layer B.Cu) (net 7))
 (segment (start 77.1101 39.0249) (end 77.1101 38.9199) (width 0.15) (layer F.Cu) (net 7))
 (segment (start 77.1101 38.9199) (end 77.55 38.48) (width 0.15) (layer F.Cu) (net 7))
 (segment (start 77.55 38.48) (end 85.83 38.48) (width 0.15) (layer F.Cu) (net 7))
 (segment (start 85.83 38.48) (end 87.630002 40.280002) (width 0.15) (layer F.Cu) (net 7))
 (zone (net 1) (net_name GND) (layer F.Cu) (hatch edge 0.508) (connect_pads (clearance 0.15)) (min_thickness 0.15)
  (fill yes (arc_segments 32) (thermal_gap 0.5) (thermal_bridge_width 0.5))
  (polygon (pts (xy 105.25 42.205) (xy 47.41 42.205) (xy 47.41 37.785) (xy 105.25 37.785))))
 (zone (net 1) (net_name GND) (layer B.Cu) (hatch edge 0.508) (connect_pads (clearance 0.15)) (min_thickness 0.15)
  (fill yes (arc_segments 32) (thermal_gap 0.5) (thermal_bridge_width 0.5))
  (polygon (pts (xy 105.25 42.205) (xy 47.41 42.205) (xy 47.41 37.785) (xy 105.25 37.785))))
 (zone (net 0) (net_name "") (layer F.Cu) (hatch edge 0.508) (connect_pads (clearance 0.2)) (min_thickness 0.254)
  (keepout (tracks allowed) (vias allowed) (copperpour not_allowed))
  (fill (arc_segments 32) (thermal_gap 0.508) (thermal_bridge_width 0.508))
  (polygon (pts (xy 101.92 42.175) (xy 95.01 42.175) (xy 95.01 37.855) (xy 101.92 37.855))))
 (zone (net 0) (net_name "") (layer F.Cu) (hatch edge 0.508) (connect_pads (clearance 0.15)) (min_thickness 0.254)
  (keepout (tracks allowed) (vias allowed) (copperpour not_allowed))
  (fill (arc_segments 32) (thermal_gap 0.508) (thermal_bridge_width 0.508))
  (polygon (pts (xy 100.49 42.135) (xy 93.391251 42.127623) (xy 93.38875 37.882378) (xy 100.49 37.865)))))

